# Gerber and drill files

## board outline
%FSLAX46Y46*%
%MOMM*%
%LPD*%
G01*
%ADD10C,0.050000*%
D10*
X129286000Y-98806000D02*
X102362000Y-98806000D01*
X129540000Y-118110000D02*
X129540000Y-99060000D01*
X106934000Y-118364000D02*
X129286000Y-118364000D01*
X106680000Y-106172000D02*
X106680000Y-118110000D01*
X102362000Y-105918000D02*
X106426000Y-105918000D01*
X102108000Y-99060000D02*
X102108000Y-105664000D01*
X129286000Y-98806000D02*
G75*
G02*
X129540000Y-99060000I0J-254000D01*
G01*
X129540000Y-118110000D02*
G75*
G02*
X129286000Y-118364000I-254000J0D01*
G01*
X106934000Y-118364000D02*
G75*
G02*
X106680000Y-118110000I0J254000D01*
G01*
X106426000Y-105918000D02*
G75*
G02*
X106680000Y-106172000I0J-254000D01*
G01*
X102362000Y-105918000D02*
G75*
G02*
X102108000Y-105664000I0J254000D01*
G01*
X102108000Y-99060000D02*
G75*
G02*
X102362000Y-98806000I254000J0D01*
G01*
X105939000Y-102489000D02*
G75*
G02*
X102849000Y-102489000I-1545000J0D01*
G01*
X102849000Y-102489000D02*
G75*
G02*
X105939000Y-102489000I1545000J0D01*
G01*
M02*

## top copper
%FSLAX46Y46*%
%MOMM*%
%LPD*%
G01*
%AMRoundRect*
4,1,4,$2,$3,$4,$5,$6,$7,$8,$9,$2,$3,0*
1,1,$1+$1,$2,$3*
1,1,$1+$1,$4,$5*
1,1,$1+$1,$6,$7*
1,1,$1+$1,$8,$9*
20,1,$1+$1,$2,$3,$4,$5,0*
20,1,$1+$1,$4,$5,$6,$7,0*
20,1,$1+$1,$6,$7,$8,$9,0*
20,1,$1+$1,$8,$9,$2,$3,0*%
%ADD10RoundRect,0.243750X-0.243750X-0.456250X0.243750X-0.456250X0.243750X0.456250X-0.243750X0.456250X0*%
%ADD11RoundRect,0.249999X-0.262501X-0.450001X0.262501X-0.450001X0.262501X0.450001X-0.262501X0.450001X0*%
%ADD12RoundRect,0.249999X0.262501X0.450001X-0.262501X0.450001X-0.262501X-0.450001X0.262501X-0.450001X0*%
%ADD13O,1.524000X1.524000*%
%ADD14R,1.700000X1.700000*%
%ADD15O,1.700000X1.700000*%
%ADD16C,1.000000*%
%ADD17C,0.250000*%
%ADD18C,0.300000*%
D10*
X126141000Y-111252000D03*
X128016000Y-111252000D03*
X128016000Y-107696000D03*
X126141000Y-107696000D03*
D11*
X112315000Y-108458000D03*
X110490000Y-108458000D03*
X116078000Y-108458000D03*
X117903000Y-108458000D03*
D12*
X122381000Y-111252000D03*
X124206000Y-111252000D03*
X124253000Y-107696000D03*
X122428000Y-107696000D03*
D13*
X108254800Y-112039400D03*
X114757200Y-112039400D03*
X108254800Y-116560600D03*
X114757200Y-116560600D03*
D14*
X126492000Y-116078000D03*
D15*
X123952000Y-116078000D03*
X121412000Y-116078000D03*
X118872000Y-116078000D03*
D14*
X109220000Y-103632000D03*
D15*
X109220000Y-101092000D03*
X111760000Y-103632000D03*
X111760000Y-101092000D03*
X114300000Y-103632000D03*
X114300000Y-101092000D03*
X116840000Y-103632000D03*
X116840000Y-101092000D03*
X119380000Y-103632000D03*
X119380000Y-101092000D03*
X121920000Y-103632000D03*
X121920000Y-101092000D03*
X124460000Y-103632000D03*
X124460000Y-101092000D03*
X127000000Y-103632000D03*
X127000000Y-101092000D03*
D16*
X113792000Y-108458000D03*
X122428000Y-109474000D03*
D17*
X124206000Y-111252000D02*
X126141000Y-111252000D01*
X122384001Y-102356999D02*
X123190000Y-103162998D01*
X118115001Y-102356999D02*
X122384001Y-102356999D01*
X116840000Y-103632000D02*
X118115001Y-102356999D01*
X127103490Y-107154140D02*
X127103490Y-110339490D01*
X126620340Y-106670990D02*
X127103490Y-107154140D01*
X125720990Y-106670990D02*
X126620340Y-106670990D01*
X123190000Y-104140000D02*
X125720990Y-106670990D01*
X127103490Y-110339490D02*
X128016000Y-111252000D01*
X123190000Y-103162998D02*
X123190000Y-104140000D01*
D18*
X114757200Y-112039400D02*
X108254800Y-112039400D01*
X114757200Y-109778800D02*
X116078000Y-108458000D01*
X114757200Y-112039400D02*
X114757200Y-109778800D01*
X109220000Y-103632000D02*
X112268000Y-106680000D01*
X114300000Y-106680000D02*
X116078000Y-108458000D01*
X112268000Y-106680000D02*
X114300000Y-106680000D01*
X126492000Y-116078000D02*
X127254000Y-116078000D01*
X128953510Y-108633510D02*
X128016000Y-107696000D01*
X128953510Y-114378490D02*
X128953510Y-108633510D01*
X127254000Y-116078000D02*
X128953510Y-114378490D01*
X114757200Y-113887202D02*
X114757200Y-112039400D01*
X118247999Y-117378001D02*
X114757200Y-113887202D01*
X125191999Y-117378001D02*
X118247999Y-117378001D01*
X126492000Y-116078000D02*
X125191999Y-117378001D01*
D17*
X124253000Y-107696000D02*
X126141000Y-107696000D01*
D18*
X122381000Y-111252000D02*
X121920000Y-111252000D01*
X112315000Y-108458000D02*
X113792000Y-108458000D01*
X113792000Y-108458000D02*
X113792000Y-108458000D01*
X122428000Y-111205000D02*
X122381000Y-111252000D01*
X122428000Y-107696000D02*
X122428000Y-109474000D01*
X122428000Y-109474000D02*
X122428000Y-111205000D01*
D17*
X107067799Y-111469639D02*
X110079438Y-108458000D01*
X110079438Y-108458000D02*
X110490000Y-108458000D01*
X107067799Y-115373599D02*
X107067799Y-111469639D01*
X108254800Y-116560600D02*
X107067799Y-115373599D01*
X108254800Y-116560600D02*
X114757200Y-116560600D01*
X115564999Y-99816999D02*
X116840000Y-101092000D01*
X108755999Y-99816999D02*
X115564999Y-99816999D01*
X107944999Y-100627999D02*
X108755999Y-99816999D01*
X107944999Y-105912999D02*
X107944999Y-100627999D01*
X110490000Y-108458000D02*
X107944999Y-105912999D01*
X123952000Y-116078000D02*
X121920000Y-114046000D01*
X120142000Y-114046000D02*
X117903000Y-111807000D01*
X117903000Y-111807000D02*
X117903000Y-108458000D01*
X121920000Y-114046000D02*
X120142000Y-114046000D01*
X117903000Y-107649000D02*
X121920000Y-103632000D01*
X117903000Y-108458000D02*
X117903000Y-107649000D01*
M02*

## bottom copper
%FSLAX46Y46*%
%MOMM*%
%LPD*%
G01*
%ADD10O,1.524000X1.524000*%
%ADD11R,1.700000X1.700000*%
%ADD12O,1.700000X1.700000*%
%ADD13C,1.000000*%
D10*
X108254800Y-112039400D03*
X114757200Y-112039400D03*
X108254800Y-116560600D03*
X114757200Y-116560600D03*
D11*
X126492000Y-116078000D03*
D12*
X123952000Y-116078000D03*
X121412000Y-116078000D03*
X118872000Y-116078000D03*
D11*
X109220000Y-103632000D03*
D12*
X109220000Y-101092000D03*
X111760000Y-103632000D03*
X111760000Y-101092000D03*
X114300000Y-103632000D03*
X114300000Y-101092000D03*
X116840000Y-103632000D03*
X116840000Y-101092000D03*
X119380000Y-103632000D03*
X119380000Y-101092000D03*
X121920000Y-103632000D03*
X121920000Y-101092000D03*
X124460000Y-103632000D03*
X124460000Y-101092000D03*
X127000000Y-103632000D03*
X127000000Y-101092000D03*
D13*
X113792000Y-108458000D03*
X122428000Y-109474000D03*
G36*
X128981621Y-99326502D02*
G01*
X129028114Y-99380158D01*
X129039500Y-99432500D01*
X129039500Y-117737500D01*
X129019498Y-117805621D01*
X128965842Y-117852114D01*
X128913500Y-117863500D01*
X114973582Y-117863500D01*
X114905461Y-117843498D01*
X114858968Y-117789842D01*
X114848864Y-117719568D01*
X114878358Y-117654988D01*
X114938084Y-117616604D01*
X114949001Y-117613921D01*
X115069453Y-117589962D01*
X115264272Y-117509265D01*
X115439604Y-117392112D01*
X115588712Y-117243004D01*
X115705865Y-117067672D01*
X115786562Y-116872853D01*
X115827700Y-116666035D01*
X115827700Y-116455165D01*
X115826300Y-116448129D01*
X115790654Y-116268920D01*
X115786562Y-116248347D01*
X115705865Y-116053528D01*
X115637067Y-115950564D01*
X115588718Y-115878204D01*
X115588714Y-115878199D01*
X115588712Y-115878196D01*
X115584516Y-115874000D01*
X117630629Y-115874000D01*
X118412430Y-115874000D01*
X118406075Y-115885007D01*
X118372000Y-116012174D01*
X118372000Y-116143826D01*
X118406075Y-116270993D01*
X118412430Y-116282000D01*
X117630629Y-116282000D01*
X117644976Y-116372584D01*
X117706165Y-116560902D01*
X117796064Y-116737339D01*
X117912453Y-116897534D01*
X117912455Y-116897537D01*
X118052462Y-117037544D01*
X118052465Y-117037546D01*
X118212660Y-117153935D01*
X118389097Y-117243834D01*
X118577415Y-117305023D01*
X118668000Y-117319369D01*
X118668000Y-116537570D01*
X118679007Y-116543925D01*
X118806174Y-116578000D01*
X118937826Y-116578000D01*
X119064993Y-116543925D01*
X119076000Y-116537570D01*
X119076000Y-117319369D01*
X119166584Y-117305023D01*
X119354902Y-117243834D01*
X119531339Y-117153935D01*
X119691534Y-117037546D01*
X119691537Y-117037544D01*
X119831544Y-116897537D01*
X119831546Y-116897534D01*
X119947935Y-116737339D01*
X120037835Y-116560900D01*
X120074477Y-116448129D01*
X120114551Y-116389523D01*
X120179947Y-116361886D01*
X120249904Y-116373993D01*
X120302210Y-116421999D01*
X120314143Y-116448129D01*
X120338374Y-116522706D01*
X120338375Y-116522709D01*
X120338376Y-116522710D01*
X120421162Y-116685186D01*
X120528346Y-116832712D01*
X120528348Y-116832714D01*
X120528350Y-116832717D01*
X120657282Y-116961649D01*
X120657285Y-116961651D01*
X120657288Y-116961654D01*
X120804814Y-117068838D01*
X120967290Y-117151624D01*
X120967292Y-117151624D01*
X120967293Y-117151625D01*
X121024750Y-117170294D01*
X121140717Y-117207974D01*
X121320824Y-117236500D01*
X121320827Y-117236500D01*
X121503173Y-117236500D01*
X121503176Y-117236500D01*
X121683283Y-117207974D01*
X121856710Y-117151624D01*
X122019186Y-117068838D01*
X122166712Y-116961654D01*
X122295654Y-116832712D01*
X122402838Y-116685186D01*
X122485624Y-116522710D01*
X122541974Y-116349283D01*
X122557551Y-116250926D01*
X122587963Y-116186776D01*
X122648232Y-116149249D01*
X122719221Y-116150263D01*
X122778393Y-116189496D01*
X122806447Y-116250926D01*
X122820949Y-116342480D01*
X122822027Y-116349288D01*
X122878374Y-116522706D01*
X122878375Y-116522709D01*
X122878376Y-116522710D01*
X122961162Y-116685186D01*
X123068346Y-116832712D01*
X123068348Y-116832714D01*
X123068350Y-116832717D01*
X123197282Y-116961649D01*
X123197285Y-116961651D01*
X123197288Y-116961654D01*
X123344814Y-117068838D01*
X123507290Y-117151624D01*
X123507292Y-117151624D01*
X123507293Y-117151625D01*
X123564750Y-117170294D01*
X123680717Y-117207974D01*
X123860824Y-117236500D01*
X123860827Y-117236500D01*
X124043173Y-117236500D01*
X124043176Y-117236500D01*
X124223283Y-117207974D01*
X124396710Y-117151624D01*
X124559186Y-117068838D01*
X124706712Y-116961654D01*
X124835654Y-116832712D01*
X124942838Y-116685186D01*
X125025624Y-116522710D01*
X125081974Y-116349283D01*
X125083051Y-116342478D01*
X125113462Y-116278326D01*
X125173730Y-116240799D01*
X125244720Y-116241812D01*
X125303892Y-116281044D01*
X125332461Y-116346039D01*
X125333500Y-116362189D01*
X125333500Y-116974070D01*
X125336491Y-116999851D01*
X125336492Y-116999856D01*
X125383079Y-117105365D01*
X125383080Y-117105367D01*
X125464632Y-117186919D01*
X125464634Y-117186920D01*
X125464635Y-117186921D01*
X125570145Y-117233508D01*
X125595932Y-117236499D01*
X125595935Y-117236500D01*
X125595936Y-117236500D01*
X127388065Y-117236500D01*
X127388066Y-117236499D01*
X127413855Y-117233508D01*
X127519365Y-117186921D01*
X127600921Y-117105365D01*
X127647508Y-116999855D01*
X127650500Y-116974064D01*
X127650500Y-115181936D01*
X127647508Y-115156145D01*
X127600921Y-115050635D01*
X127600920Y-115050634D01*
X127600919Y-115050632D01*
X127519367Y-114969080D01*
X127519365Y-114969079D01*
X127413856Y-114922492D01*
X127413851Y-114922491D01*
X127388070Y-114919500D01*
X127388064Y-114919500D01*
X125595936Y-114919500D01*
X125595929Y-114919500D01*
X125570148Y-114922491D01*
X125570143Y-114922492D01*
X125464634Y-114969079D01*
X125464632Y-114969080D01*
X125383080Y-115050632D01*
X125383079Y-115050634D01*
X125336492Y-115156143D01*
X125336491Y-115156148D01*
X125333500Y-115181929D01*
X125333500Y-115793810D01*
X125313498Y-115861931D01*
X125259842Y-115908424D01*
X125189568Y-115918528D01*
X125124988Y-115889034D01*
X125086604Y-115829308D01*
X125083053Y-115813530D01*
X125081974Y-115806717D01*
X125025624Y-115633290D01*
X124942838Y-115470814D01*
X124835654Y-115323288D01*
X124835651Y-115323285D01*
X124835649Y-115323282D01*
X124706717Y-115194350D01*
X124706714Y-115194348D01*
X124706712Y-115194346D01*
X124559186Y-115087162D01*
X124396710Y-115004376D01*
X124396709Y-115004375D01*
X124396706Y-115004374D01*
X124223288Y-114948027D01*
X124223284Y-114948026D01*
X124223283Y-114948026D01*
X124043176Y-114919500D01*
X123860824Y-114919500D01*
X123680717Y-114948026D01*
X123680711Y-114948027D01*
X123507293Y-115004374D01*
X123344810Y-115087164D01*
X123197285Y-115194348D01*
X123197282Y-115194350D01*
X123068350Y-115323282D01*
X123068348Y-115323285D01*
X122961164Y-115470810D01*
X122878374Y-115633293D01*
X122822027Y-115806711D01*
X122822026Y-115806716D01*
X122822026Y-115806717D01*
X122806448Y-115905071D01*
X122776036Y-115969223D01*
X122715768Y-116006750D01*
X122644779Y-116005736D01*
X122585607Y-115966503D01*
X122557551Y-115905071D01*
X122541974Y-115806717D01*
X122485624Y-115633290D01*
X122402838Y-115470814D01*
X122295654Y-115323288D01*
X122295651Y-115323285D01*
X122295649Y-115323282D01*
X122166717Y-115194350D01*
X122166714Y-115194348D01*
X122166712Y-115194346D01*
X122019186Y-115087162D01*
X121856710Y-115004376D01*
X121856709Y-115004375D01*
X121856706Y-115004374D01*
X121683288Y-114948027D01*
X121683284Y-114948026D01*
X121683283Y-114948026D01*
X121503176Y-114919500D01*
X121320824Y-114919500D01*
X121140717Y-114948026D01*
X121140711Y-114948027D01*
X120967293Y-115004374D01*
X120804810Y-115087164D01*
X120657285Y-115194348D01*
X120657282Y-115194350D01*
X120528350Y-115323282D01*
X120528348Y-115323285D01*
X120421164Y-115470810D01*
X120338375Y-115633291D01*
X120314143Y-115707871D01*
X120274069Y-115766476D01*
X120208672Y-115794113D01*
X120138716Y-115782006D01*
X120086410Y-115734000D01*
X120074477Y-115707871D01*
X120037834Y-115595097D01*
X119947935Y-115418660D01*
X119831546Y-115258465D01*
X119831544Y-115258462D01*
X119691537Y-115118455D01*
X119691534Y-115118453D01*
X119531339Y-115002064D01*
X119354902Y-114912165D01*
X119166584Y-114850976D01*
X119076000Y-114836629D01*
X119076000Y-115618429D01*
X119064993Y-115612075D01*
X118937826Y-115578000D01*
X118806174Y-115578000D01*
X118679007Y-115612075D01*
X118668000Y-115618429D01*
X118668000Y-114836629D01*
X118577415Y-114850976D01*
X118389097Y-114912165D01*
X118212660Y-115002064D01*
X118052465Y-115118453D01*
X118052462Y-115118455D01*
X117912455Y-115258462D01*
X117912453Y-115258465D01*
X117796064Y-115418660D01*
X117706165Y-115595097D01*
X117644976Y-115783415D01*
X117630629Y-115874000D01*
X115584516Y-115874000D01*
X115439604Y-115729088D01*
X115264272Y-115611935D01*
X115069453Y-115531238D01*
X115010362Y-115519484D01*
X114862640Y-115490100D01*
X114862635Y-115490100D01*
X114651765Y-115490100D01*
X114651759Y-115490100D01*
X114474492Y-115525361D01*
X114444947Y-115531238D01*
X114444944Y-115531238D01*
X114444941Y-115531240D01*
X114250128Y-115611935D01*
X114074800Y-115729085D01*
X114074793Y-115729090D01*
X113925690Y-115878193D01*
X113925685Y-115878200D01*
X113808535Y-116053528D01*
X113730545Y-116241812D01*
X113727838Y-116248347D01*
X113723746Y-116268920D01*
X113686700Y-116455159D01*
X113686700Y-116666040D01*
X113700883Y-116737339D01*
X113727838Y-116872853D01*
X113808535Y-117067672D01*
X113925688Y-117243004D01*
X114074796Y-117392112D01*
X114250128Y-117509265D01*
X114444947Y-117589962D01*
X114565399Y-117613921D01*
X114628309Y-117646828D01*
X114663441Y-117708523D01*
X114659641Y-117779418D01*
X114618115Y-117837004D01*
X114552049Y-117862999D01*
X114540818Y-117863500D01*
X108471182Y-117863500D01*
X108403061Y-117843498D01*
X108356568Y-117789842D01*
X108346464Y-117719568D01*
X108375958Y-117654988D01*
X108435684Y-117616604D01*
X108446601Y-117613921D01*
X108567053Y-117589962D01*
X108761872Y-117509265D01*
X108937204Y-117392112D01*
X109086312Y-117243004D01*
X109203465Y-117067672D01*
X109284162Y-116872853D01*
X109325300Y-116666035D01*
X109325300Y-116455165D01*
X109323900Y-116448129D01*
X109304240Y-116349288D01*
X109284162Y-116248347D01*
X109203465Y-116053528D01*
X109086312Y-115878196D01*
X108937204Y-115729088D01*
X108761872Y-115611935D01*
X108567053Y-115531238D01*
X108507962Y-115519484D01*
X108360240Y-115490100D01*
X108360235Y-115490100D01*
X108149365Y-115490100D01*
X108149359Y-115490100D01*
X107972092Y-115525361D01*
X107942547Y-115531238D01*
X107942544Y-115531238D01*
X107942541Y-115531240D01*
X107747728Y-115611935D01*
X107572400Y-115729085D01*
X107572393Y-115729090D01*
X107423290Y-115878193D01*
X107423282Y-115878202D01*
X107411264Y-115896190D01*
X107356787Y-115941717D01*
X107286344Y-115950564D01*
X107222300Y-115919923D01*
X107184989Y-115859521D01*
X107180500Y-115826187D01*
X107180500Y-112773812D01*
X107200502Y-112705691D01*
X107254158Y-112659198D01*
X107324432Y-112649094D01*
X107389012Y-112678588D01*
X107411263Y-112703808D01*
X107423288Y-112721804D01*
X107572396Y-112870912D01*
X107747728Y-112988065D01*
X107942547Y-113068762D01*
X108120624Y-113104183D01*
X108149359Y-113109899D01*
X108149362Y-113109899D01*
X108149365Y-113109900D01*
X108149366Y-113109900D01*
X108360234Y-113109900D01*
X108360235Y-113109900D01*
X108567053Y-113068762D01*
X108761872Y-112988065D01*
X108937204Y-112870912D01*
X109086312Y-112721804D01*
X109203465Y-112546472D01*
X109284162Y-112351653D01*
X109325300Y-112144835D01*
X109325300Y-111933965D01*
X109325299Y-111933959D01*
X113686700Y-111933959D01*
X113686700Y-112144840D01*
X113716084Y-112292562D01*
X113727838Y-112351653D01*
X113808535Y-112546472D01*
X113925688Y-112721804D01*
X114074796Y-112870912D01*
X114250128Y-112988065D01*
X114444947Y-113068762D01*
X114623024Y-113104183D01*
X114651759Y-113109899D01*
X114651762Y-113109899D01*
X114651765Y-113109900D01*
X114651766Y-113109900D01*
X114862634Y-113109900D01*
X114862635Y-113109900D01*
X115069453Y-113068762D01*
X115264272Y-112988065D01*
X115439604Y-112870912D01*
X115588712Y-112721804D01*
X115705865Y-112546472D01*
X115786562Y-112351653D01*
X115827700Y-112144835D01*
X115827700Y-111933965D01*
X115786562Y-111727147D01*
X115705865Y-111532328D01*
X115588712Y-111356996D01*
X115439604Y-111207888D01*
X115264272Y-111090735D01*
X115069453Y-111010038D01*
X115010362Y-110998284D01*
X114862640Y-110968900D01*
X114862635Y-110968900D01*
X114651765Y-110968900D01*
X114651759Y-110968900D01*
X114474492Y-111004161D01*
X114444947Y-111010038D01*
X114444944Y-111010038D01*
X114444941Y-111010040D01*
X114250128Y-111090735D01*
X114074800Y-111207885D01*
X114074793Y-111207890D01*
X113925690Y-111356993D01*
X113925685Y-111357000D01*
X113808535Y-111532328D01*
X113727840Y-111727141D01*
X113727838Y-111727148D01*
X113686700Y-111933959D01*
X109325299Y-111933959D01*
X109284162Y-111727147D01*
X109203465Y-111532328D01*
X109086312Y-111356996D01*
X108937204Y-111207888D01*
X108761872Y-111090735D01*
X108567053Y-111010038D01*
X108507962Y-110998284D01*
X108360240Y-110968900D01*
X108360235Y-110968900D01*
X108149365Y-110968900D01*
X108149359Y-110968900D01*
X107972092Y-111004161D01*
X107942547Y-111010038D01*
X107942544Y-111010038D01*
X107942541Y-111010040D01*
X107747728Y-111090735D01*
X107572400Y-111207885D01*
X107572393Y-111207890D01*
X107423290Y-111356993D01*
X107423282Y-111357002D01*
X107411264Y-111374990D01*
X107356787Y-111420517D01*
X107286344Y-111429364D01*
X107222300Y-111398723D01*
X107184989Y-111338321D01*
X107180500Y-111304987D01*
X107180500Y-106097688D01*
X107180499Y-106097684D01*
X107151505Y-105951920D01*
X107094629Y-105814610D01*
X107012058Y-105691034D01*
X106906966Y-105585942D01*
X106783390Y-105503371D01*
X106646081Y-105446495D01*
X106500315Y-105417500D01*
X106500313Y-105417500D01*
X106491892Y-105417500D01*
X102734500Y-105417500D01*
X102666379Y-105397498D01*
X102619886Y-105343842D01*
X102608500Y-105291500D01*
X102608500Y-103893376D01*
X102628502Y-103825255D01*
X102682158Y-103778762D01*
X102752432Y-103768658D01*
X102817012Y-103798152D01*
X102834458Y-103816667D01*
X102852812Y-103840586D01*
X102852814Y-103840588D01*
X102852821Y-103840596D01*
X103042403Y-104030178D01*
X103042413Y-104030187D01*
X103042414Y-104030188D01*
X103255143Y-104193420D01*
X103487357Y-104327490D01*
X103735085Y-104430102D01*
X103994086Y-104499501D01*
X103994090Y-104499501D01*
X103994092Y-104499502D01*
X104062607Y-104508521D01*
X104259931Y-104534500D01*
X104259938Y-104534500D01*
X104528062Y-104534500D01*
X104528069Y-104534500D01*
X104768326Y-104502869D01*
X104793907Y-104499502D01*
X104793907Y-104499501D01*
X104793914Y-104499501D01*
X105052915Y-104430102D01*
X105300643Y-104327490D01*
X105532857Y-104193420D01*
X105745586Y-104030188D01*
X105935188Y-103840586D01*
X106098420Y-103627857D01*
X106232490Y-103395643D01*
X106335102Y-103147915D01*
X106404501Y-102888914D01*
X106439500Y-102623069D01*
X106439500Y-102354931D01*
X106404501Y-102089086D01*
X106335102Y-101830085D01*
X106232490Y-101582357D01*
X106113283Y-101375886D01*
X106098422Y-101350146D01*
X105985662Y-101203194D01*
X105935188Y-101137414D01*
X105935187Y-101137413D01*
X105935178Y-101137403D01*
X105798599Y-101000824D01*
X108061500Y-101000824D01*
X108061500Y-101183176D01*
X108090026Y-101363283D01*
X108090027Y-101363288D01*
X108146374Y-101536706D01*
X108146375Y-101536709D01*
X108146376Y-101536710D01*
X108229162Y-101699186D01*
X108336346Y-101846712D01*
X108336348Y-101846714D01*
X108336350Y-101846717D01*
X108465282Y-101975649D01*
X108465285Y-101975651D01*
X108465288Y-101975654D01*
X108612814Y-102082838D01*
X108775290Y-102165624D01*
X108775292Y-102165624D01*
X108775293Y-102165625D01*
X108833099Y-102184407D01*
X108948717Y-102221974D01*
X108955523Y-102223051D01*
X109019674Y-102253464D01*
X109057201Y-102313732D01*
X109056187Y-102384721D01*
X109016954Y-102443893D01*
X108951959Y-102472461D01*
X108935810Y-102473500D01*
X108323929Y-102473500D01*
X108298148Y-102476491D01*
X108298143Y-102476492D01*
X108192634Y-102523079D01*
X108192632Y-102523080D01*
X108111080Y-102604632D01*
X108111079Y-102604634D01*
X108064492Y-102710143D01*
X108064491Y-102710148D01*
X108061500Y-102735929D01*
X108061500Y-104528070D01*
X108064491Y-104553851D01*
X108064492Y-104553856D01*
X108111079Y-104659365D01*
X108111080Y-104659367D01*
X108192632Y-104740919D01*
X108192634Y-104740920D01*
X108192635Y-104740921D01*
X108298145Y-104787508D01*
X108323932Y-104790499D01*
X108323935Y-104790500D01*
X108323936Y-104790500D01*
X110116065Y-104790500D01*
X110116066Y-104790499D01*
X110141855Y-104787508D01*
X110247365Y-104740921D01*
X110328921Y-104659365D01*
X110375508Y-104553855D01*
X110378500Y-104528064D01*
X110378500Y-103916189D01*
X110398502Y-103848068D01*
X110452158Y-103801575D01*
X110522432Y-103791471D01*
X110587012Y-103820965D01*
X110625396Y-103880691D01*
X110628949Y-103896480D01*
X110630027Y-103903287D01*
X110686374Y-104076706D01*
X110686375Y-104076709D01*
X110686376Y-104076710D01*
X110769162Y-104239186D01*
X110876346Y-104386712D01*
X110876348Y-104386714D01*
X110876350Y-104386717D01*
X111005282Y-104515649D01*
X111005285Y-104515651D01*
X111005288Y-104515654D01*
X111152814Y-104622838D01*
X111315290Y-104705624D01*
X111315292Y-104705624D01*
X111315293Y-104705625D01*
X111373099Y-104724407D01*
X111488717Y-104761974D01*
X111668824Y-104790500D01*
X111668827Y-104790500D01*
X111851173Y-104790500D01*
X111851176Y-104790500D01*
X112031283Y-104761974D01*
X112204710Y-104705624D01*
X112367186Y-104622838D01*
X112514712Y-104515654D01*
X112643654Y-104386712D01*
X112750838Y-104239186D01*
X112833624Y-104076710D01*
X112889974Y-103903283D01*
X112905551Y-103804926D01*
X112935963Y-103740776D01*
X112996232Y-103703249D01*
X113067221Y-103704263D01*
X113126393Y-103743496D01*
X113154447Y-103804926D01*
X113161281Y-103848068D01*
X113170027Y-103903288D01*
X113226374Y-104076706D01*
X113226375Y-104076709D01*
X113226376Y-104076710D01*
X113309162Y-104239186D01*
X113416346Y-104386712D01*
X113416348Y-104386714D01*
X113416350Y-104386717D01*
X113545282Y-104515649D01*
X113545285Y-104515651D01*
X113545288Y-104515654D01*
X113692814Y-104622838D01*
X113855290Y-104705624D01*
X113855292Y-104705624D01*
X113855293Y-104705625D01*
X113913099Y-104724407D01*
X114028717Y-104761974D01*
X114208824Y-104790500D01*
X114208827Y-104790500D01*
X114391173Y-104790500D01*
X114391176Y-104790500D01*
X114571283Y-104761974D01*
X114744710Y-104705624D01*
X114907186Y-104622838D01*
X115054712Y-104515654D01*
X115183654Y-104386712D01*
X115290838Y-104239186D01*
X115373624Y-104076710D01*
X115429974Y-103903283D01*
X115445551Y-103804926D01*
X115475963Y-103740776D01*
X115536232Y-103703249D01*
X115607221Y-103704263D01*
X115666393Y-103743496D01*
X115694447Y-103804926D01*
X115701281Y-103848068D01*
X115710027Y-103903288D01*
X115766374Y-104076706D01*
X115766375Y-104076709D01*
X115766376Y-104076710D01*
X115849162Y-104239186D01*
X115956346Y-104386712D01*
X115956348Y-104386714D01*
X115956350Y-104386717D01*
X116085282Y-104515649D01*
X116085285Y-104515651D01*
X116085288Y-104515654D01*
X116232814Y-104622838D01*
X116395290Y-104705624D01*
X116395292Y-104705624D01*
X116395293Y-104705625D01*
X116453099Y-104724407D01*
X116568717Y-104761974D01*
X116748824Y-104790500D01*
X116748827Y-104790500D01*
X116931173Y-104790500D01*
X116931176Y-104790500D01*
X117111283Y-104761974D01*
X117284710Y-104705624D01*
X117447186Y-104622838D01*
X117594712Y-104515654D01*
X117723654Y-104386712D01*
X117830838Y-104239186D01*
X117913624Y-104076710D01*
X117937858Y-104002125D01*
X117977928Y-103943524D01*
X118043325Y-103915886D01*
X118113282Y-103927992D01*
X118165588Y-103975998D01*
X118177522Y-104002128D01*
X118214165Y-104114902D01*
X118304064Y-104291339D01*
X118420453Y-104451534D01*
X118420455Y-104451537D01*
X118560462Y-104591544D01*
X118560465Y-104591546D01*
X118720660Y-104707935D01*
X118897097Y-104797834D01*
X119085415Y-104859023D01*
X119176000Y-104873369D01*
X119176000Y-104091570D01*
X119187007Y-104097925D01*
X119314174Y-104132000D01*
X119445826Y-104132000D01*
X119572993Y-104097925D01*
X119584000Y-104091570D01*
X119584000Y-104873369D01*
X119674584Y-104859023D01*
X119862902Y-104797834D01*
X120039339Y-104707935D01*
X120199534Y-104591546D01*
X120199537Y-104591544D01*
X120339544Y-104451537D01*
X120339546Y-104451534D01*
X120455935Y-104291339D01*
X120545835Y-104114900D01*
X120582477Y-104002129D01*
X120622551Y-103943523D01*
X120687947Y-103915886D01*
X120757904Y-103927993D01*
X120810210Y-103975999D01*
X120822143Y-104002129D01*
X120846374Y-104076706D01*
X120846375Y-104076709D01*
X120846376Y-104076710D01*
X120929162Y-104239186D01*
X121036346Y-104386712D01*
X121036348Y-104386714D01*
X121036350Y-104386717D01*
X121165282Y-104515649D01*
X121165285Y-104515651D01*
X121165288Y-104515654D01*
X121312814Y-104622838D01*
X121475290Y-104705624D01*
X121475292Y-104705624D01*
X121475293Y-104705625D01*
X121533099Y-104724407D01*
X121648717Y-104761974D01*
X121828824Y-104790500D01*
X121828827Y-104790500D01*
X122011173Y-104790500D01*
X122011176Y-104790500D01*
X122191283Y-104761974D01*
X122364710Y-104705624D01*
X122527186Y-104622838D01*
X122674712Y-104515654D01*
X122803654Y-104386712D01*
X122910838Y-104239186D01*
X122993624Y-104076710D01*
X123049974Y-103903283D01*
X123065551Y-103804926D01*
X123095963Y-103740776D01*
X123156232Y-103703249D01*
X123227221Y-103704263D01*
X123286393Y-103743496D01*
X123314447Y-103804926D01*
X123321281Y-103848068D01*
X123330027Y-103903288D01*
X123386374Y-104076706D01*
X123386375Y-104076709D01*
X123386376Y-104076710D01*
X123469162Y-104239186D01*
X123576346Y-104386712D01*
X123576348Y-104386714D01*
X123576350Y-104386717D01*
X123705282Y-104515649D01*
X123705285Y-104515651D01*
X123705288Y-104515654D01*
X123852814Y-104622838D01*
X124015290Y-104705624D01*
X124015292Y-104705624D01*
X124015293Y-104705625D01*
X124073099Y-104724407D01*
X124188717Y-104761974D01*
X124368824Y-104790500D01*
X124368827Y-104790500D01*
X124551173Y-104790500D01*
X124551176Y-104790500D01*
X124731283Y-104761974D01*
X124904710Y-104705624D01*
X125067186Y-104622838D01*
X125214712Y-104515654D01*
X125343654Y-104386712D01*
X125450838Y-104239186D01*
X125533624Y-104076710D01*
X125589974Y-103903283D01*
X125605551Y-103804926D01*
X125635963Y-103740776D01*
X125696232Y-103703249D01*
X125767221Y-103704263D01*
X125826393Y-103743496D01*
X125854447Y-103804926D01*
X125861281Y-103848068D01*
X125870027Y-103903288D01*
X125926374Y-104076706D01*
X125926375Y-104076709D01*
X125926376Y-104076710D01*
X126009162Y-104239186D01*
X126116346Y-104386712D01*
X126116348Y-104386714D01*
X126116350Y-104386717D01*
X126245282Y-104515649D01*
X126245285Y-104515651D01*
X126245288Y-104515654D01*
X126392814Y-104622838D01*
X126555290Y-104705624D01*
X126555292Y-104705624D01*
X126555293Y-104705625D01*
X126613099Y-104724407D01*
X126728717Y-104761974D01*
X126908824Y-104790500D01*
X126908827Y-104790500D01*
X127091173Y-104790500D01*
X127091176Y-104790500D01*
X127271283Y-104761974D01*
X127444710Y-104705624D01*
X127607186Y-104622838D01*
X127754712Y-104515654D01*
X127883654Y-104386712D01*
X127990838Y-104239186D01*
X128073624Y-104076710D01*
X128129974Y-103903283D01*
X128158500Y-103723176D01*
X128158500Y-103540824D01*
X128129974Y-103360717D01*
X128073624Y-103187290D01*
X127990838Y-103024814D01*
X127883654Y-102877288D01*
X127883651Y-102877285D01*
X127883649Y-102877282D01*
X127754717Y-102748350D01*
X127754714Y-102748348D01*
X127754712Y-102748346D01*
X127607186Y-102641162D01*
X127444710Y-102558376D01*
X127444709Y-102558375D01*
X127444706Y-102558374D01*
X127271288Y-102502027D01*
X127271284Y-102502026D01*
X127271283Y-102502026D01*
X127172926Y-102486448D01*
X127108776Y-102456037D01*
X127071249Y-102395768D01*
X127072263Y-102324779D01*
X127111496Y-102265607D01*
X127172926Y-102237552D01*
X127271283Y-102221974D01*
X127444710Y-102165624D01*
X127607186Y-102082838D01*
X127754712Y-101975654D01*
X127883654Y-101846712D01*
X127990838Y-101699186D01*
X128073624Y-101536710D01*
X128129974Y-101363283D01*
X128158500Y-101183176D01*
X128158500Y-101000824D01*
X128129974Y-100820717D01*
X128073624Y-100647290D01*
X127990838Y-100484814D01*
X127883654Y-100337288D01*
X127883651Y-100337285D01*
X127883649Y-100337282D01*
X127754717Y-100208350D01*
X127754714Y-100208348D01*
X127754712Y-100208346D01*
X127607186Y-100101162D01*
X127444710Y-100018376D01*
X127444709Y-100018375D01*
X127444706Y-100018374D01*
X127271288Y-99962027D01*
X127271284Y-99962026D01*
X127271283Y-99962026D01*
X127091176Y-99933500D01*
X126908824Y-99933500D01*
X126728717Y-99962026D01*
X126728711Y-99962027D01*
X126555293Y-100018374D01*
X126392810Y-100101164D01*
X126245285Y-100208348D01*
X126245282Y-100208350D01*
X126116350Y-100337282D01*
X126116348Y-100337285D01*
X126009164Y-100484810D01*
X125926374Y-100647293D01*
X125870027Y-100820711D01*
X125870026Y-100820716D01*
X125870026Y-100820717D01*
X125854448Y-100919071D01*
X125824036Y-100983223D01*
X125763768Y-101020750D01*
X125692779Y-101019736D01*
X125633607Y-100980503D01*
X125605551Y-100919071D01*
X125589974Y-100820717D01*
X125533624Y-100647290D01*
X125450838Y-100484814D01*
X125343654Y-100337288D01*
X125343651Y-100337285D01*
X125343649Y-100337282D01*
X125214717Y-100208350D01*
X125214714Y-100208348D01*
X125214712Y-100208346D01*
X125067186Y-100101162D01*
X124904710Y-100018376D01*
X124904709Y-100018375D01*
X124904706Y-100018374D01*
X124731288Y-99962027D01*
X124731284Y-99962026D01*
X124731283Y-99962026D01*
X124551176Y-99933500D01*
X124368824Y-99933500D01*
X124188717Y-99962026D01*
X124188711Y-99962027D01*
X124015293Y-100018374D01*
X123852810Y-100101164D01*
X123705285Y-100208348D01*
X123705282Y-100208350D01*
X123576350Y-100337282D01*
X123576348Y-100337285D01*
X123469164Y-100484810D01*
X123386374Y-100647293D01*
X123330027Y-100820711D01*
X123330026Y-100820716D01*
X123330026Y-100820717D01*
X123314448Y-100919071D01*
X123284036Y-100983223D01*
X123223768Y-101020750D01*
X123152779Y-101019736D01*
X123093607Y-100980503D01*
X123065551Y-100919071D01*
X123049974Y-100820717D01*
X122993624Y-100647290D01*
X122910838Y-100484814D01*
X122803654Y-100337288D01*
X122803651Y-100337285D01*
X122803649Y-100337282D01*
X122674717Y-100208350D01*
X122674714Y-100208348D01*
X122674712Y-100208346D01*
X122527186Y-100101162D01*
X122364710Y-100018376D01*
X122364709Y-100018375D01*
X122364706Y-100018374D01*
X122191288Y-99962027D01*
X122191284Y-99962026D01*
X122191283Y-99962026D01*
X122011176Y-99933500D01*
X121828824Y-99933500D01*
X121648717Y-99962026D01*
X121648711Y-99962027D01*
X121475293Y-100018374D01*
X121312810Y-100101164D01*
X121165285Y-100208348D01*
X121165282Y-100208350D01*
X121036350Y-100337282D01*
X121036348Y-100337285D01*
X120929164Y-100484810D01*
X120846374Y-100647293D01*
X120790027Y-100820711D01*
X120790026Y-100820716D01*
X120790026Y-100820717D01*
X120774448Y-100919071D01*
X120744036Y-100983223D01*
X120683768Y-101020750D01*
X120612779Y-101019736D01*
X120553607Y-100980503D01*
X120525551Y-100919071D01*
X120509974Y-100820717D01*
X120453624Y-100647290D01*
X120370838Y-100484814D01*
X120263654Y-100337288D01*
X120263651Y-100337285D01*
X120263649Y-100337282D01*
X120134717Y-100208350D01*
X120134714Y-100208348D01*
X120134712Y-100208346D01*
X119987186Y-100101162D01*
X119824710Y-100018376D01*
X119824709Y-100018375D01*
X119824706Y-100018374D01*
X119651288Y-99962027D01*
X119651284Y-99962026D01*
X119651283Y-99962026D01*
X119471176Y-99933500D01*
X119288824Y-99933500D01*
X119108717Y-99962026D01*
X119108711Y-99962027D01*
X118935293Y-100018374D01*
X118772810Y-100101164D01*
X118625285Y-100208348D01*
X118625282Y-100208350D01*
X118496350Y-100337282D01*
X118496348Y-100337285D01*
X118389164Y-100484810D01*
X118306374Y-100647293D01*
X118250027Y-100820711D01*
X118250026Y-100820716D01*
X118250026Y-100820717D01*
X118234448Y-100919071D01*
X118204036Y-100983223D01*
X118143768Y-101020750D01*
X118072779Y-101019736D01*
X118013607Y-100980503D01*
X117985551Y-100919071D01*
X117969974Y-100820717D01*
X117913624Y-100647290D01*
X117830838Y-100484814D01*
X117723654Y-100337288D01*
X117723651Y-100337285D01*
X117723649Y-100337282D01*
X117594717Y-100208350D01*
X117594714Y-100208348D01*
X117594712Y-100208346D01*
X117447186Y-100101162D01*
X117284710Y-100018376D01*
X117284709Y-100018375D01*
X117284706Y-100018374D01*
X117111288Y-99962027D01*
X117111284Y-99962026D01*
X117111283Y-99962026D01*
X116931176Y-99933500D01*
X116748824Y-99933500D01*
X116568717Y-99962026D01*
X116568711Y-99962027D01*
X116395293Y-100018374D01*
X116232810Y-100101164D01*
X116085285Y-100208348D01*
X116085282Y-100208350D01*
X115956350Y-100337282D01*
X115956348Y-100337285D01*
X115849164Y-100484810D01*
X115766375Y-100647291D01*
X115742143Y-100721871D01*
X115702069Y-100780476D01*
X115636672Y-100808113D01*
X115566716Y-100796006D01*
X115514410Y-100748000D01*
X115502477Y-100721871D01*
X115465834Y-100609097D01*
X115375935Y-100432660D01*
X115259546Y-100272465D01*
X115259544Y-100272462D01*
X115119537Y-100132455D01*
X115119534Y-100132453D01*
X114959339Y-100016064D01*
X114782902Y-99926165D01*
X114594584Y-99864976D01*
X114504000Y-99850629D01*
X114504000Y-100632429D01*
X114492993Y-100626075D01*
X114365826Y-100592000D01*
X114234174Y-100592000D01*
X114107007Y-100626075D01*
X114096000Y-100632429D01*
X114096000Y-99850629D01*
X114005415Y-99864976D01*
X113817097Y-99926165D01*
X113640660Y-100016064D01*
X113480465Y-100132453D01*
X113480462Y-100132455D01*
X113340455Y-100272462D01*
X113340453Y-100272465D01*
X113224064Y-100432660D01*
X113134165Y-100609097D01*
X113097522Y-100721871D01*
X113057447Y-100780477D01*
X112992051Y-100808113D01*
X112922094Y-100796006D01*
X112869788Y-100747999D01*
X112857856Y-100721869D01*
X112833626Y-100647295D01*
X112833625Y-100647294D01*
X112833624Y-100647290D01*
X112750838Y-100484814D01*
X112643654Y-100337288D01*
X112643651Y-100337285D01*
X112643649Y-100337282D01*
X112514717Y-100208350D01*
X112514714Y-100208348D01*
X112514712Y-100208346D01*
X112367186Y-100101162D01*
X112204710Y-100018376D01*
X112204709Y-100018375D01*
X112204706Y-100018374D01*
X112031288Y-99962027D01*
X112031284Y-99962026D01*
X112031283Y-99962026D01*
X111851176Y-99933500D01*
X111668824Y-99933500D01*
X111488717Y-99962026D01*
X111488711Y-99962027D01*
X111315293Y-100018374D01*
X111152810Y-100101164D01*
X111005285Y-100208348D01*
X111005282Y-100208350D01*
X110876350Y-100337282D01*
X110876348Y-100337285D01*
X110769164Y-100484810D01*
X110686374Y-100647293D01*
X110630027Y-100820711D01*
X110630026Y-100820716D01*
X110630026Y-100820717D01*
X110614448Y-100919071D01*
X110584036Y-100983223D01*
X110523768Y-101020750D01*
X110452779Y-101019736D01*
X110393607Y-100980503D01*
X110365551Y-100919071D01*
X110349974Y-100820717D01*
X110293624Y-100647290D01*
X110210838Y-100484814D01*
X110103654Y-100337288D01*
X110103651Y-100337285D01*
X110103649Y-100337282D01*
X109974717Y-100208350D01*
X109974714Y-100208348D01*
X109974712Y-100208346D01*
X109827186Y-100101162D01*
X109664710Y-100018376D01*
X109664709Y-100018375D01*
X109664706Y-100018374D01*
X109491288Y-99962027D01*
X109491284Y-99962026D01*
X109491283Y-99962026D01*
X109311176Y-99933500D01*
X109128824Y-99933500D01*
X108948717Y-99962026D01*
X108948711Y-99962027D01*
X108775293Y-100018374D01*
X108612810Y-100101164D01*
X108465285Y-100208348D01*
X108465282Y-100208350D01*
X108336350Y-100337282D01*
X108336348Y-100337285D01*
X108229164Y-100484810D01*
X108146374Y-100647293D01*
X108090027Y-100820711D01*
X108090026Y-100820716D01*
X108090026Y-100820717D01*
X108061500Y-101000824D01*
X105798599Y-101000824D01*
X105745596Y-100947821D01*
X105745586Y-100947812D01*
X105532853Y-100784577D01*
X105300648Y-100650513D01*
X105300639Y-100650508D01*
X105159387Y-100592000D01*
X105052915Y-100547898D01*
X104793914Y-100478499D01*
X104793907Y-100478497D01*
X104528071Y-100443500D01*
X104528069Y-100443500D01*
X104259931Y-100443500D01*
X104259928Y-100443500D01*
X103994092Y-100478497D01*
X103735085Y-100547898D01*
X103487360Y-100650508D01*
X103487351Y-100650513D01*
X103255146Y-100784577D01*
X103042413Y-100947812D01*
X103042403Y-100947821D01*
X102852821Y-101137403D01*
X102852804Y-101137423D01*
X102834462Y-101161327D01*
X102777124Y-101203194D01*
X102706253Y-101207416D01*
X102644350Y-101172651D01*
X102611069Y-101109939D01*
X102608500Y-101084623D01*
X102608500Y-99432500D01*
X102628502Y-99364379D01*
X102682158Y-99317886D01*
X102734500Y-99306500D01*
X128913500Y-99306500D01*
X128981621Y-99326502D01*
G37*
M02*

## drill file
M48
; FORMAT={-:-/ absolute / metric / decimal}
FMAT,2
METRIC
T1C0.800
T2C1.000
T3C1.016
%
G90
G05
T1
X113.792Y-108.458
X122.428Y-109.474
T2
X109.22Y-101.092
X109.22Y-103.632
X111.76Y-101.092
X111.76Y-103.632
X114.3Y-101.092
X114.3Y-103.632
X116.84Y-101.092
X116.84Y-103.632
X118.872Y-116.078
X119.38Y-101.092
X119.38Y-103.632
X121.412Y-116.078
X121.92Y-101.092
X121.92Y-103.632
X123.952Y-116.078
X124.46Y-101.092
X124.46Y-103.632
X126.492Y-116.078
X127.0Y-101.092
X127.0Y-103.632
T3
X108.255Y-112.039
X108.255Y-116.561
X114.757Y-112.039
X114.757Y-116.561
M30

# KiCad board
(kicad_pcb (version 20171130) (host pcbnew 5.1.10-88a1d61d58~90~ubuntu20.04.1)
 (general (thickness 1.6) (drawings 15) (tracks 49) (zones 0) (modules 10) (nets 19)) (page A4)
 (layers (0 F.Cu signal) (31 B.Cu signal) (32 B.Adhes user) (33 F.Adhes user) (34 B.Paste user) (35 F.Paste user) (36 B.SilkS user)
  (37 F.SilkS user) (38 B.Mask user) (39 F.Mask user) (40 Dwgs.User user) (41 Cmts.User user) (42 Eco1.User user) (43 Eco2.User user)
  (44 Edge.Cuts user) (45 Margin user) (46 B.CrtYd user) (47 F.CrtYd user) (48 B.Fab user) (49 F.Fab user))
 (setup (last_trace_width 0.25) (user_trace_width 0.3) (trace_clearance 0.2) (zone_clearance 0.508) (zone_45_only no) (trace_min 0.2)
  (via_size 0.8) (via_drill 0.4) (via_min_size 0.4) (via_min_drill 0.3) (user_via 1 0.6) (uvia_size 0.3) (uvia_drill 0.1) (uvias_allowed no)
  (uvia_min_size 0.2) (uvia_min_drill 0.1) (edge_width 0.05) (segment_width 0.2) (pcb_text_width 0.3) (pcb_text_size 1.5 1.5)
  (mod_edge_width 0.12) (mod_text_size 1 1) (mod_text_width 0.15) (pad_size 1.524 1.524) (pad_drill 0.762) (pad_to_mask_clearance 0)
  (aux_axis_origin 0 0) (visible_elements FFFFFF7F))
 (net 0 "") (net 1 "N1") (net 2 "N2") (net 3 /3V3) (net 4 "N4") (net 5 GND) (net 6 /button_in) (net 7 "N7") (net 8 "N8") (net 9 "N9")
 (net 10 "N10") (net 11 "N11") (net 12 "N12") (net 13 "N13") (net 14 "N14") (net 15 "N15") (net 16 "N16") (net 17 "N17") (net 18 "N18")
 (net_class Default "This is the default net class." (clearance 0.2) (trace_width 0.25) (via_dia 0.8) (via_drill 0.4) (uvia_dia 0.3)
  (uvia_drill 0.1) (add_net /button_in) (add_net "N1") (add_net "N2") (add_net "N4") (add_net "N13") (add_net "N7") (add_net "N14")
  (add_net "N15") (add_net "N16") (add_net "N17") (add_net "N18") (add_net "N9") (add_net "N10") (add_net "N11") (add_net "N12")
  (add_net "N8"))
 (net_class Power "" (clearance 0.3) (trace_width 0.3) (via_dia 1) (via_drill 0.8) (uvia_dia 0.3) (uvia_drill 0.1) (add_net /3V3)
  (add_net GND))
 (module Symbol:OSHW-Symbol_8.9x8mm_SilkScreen (layer B.Cu) (at 123.698 109.22)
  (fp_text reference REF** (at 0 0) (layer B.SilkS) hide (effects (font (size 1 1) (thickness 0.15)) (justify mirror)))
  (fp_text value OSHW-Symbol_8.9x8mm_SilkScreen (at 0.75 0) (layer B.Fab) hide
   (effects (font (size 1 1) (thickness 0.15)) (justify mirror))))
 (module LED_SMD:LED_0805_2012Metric (layer F.Cu) (at 127.0785 111.252)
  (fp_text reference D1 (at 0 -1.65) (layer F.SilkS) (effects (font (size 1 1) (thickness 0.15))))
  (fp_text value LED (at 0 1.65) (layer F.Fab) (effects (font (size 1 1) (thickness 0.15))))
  (pad 1 smd roundrect (at -0.9375 0) (size 0.975 1.4) (layers F.Cu F.Paste F.Mask) (roundrect_rratio 0.25) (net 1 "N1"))
  (pad 2 smd roundrect (at 0.9375 0) (size 0.975 1.4) (layers F.Cu F.Paste F.Mask) (roundrect_rratio 0.25) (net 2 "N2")))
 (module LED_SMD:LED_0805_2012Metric (layer F.Cu) (at 127.0785 107.696)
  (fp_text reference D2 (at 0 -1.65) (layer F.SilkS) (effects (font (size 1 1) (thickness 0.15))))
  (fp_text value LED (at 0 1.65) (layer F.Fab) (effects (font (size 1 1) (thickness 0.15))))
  (pad 2 smd roundrect (at 0.9375 0) (size 0.975 1.4) (layers F.Cu F.Paste F.Mask) (roundrect_rratio 0.25) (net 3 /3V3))
  (pad 1 smd roundrect (at -0.9375 0) (size 0.975 1.4) (layers F.Cu F.Paste F.Mask) (roundrect_rratio 0.25) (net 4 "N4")))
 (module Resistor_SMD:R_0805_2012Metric (layer F.Cu) (at 111.4025 108.458)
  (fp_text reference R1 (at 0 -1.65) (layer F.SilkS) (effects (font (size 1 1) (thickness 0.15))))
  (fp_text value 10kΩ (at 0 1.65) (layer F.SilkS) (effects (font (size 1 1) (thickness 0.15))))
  (pad 2 smd roundrect (at 0.9125 0) (size 1.025 1.4) (layers F.Cu F.Paste F.Mask) (roundrect_rratio 0.2439014634146341) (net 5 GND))
  (pad 1 smd roundrect (at -0.9125 0) (size 1.025 1.4) (layers F.Cu F.Paste F.Mask) (roundrect_rratio 0.2439014634146341) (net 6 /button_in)))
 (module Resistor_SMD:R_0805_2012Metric (layer F.Cu) (at 116.9905 108.458)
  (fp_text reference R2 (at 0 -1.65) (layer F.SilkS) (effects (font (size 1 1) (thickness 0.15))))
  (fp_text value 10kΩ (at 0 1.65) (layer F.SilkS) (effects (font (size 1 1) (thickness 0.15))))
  (pad 1 smd roundrect (at -0.9125 0) (size 1.025 1.4) (layers F.Cu F.Paste F.Mask) (roundrect_rratio 0.2439014634146341) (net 3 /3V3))
  (pad 2 smd roundrect (at 0.9125 0) (size 1.025 1.4) (layers F.Cu F.Paste F.Mask) (roundrect_rratio 0.2439014634146341) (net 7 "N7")))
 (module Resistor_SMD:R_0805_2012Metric (layer F.Cu) (at 123.2935 111.252 180)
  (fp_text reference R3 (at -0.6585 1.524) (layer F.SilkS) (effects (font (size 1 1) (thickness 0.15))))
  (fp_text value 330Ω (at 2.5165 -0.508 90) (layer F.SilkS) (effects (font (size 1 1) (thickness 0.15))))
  (pad 2 smd roundrect (at 0.9125 0 180) (size 1.025 1.4) (layers F.Cu F.Paste F.Mask) (roundrect_rratio 0.2439014634146341) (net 5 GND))
  (pad 1 smd roundrect (at -0.9125 0 180) (size 1.025 1.4) (layers F.Cu F.Paste F.Mask) (roundrect_rratio 0.2439014634146341) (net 1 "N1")))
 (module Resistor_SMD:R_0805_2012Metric (layer F.Cu) (at 123.3405 107.696 180)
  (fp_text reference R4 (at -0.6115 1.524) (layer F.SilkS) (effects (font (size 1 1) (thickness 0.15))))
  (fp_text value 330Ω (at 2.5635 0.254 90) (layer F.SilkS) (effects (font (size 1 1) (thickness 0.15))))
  (pad 1 smd roundrect (at -0.9125 0 180) (size 1.025 1.4) (layers F.Cu F.Paste F.Mask) (roundrect_rratio 0.2439014634146341) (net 4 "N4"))
  (pad 2 smd roundrect (at 0.9125 0 180) (size 1.025 1.4) (layers F.Cu F.Paste F.Mask) (roundrect_rratio 0.2439014634146341) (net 5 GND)))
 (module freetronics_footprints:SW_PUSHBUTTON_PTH (layer F.Cu) (at 111.506 114.3)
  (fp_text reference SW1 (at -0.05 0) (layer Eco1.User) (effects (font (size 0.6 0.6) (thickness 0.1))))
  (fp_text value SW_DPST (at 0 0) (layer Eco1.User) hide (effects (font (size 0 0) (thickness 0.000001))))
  (pad 1 thru_hole oval (at -3.2512 -2.2606) (size 1.524 1.524) (drill 1.016) (layers *.Cu *.Mask) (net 3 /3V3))
  (pad 1 thru_hole oval (at 3.2512 -2.2606) (size 1.524 1.524) (drill 1.016) (layers *.Cu *.Mask) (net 3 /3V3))
  (pad 2 thru_hole oval (at -3.2512 2.2606) (size 1.524 1.524) (drill 1.016) (layers *.Cu *.Mask) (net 6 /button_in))
  (pad 2 thru_hole oval (at 3.2512 2.2606) (size 1.524 1.524) (drill 1.016) (layers *.Cu *.Mask) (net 6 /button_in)))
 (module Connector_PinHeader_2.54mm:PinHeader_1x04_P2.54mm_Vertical (layer F.Cu) (at 126.492 116.078 270)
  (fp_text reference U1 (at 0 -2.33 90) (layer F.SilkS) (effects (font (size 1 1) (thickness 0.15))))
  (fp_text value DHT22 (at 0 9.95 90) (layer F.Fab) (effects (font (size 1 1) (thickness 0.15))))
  (pad 1 thru_hole rect (at 0 0 270) (size 1.7 1.7) (drill 1) (layers *.Cu *.Mask) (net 3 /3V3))
  (pad 2 thru_hole oval (at 0 2.54 270) (size 1.7 1.7) (drill 1) (layers *.Cu *.Mask) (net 7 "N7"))
  (pad 3 thru_hole oval (at 0 5.08 270) (size 1.7 1.7) (drill 1) (layers *.Cu *.Mask) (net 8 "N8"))
  (pad 4 thru_hole oval (at 0 7.62 270) (size 1.7 1.7) (drill 1) (layers *.Cu *.Mask) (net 5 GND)))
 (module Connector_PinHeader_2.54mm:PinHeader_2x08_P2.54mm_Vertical (layer F.Cu) (at 109.22 103.632 90)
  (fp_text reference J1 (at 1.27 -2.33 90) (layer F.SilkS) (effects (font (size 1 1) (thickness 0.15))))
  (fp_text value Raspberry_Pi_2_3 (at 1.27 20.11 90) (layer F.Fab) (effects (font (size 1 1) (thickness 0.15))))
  (pad 1 thru_hole rect (at 0 0 90) (size 1.7 1.7) (drill 1) (layers *.Cu *.Mask) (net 3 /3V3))
  (pad 2 thru_hole oval (at 2.54 0 90) (size 1.7 1.7) (drill 1) (layers *.Cu *.Mask) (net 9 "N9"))
  (pad 3 thru_hole oval (at 0 2.54 90) (size 1.7 1.7) (drill 1) (layers *.Cu *.Mask) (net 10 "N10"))
  (pad 4 thru_hole oval (at 2.54 2.54 90) (size 1.7 1.7) (drill 1) (layers *.Cu *.Mask) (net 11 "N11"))
  (pad 5 thru_hole oval (at 0 5.08 90) (size 1.7 1.7) (drill 1) (layers *.Cu *.Mask) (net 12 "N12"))
  (pad 6 thru_hole oval (at 2.54 5.08 90) (size 1.7 1.7) (drill 1) (layers *.Cu *.Mask) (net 5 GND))
  (pad 7 thru_hole oval (at 0 7.62 90) (size 1.7 1.7) (drill 1) (layers *.Cu *.Mask) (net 2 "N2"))
  (pad 8 thru_hole oval (at 2.54 7.62 90) (size 1.7 1.7) (drill 1) (layers *.Cu *.Mask) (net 6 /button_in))
  (pad 9 thru_hole oval (at 0 10.16 90) (size 1.7 1.7) (drill 1) (layers *.Cu *.Mask) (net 5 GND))
  (pad 10 thru_hole oval (at 2.54 10.16 90) (size 1.7 1.7) (drill 1) (layers *.Cu *.Mask) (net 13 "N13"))
  (pad 11 thru_hole oval (at 0 12.7 90) (size 1.7 1.7) (drill 1) (layers *.Cu *.Mask) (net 7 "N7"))
  (pad 12 thru_hole oval (at 2.54 12.7 90) (size 1.7 1.7) (drill 1) (layers *.Cu *.Mask) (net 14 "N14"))
  (pad 13 thru_hole oval (at 0 15.24 90) (size 1.7 1.7) (drill 1) (layers *.Cu *.Mask) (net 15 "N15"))
  (pad 14 thru_hole oval (at 2.54 15.24 90) (size 1.7 1.7) (drill 1) (layers *.Cu *.Mask) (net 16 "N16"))
  (pad 15 thru_hole oval (at 0 17.78 90) (size 1.7 1.7) (drill 1) (layers *.Cu *.Mask) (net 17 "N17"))
  (pad 16 thru_hole oval (at 2.54 17.78 90) (size 1.7 1.7) (drill 1) (layers *.Cu *.Mask) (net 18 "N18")))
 (gr_line (start 129.286 98.806) (end 102.362 98.806) (layer Edge.Cuts) (width 0.05))
 (gr_line (start 129.54 118.11) (end 129.54 99.06) (layer Edge.Cuts) (width 0.05))
 (gr_line (start 106.934 118.364) (end 129.286 118.364) (layer Edge.Cuts) (width 0.05))
 (gr_line (start 106.68 106.172) (end 106.68 118.11) (layer Edge.Cuts) (width 0.05))
 (gr_line (start 102.362 105.918) (end 106.426 105.918) (layer Edge.Cuts) (width 0.05))
 (gr_line (start 102.108 99.06) (end 102.108 105.664) (layer Edge.Cuts) (width 0.05))
 (gr_arc (start 129.286 99.06) (end 129.54 99.06) (angle -90) (layer Edge.Cuts) (width 0.05))
 (gr_arc (start 129.286 118.11) (end 129.286 118.364) (angle -90) (layer Edge.Cuts) (width 0.05))
 (gr_arc (start 106.934 118.11) (end 106.68 118.11) (angle -90) (layer Edge.Cuts) (width 0.05))
 (gr_arc (start 106.426 106.172) (end 106.68 106.172) (angle -90) (layer Edge.Cuts) (width 0.05))
 (gr_arc (start 102.362 105.664) (end 102.108 105.664) (angle -90) (layer Edge.Cuts) (width 0.05))
 (gr_arc (start 102.362 99.06) (end 102.362 98.806) (angle -90) (layer Edge.Cuts) (width 0.05))
 (gr_circle (center 104.394 102.489) (end 105.939 102.489) (layer Edge.Cuts) (width 0.05))
 (segment (start 124.206 111.252) (end 126.141 111.252) (width 0.25) (layer F.Cu) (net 1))
 (segment (start 122.384001 102.356999) (end 123.19 103.162998) (width 0.25) (layer F.Cu) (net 2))
 (segment (start 118.115001 102.356999) (end 122.384001 102.356999) (width 0.25) (layer F.Cu) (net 2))
 (segment (start 116.84 103.632) (end 118.115001 102.356999) (width 0.25) (layer F.Cu) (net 2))
 (segment (start 127.10349 107.15414) (end 127.10349 110.33949) (width 0.25) (layer F.Cu) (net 2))
 (segment (start 126.62034 106.67099) (end 127.10349 107.15414) (width 0.25) (layer F.Cu) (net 2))
 (segment (start 125.72099 106.67099) (end 126.62034 106.67099) (width 0.25) (layer F.Cu) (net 2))
 (segment (start 123.19 104.14) (end 125.72099 106.67099) (width 0.25) (layer F.Cu) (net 2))
 (segment (start 127.10349 110.33949) (end 128.016 111.252) (width 0.25) (layer F.Cu) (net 2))
 (segment (start 123.19 103.162998) (end 123.19 104.14) (width 0.25) (layer F.Cu) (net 2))
 (segment (start 114.7572 112.0394) (end 108.2548 112.0394) (width 0.3) (layer F.Cu) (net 3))
 (segment (start 114.7572 109.7788) (end 116.078 108.458) (width 0.3) (layer F.Cu) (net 3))
 (segment (start 114.7572 112.0394) (end 114.7572 109.7788) (width 0.3) (layer F.Cu) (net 3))
 (segment (start 109.22 103.632) (end 112.268 106.68) (width 0.3) (layer F.Cu) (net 3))
 (segment (start 114.3 106.68) (end 116.078 108.458) (width 0.3) (layer F.Cu) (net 3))
 (segment (start 112.268 106.68) (end 114.3 106.68) (width 0.3) (layer F.Cu) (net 3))
 (segment (start 126.492 116.078) (end 127.254 116.078) (width 0.3) (layer F.Cu) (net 3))
 (segment (start 128.95351 108.63351) (end 128.016 107.696) (width 0.3) (layer F.Cu) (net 3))
 (segment (start 128.95351 114.37849) (end 128.95351 108.63351) (width 0.3) (layer F.Cu) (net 3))
 (segment (start 127.254 116.078) (end 128.95351 114.37849) (width 0.3) (layer F.Cu) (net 3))
 (segment (start 114.7572 113.887202) (end 114.7572 112.0394) (width 0.3) (layer F.Cu) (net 3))
 (segment (start 118.247999 117.378001) (end 114.7572 113.887202) (width 0.3) (layer F.Cu) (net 3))
 (segment (start 125.191999 117.378001) (end 118.247999 117.378001) (width 0.3) (layer F.Cu) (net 3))
 (segment (start 126.492 116.078) (end 125.191999 117.378001) (width 0.3) (layer F.Cu) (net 3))
 (segment (start 124.253 107.696) (end 126.141 107.696) (width 0.25) (layer F.Cu) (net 4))
 (segment (start 122.381 111.252) (end 121.92 111.252) (width 0.3) (layer F.Cu) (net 5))
 (segment (start 112.315 108.458) (end 113.792 108.458) (width 0.3) (layer F.Cu) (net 5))
 (segment (start 113.792 108.458) (end 113.792 108.458) (width 0.3) (layer F.Cu) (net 5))
 (via (at 113.792 108.458) (size 1) (drill 0.8) (layers F.Cu B.Cu) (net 5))
 (segment (start 122.428 111.205) (end 122.381 111.252) (width 0.3) (layer F.Cu) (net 5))
 (segment (start 122.428 107.696) (end 122.428 109.474) (width 0.3) (layer F.Cu) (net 5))
 (segment (start 122.428 109.474) (end 122.428 111.205) (width 0.3) (layer F.Cu) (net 5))
 (via (at 122.428 109.474) (size 1) (drill 0.8) (layers F.Cu B.Cu) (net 5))
 (segment (start 107.067799 111.469639) (end 110.079438 108.458) (width 0.25) (layer F.Cu) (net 6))
 (segment (start 110.079438 108.458) (end 110.49 108.458) (width 0.25) (layer F.Cu) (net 6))
 (segment (start 107.067799 115.373599) (end 107.067799 111.469639) (width 0.25) (layer F.Cu) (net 6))
 (segment (start 108.2548 116.5606) (end 107.067799 115.373599) (width 0.25) (layer F.Cu) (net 6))
 (segment (start 108.2548 116.5606) (end 114.7572 116.5606) (width 0.25) (layer F.Cu) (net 6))
 (segment (start 115.564999 99.816999) (end 116.84 101.092) (width 0.25) (layer F.Cu) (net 6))
 (segment (start 108.755999 99.816999) (end 115.564999 99.816999) (width 0.25) (layer F.Cu) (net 6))
 (segment (start 107.944999 100.627999) (end 108.755999 99.816999) (width 0.25) (layer F.Cu) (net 6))
 (segment (start 107.944999 105.912999) (end 107.944999 100.627999) (width 0.25) (layer F.Cu) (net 6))
 (segment (start 110.49 108.458) (end 107.944999 105.912999) (width 0.25) (layer F.Cu) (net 6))
 (segment (start 123.952 116.078) (end 121.92 114.046) (width 0.25) (layer F.Cu) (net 7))
 (segment (start 120.142 114.046) (end 117.903 111.807) (width 0.25) (layer F.Cu) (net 7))
 (segment (start 117.903 111.807) (end 117.903 108.458) (width 0.25) (layer F.Cu) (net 7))
 (segment (start 121.92 114.046) (end 120.142 114.046) (width 0.25) (layer F.Cu) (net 7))
 (segment (start 117.903 107.649) (end 121.92 103.632) (width 0.25) (layer F.Cu) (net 7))
 (segment (start 117.903 108.458) (end 117.903 107.649) (width 0.25) (layer F.Cu) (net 7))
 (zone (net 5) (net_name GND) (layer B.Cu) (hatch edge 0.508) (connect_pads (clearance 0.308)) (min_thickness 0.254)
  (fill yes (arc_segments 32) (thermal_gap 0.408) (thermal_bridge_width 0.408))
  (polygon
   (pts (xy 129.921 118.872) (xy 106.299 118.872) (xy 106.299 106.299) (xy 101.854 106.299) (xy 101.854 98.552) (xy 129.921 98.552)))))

